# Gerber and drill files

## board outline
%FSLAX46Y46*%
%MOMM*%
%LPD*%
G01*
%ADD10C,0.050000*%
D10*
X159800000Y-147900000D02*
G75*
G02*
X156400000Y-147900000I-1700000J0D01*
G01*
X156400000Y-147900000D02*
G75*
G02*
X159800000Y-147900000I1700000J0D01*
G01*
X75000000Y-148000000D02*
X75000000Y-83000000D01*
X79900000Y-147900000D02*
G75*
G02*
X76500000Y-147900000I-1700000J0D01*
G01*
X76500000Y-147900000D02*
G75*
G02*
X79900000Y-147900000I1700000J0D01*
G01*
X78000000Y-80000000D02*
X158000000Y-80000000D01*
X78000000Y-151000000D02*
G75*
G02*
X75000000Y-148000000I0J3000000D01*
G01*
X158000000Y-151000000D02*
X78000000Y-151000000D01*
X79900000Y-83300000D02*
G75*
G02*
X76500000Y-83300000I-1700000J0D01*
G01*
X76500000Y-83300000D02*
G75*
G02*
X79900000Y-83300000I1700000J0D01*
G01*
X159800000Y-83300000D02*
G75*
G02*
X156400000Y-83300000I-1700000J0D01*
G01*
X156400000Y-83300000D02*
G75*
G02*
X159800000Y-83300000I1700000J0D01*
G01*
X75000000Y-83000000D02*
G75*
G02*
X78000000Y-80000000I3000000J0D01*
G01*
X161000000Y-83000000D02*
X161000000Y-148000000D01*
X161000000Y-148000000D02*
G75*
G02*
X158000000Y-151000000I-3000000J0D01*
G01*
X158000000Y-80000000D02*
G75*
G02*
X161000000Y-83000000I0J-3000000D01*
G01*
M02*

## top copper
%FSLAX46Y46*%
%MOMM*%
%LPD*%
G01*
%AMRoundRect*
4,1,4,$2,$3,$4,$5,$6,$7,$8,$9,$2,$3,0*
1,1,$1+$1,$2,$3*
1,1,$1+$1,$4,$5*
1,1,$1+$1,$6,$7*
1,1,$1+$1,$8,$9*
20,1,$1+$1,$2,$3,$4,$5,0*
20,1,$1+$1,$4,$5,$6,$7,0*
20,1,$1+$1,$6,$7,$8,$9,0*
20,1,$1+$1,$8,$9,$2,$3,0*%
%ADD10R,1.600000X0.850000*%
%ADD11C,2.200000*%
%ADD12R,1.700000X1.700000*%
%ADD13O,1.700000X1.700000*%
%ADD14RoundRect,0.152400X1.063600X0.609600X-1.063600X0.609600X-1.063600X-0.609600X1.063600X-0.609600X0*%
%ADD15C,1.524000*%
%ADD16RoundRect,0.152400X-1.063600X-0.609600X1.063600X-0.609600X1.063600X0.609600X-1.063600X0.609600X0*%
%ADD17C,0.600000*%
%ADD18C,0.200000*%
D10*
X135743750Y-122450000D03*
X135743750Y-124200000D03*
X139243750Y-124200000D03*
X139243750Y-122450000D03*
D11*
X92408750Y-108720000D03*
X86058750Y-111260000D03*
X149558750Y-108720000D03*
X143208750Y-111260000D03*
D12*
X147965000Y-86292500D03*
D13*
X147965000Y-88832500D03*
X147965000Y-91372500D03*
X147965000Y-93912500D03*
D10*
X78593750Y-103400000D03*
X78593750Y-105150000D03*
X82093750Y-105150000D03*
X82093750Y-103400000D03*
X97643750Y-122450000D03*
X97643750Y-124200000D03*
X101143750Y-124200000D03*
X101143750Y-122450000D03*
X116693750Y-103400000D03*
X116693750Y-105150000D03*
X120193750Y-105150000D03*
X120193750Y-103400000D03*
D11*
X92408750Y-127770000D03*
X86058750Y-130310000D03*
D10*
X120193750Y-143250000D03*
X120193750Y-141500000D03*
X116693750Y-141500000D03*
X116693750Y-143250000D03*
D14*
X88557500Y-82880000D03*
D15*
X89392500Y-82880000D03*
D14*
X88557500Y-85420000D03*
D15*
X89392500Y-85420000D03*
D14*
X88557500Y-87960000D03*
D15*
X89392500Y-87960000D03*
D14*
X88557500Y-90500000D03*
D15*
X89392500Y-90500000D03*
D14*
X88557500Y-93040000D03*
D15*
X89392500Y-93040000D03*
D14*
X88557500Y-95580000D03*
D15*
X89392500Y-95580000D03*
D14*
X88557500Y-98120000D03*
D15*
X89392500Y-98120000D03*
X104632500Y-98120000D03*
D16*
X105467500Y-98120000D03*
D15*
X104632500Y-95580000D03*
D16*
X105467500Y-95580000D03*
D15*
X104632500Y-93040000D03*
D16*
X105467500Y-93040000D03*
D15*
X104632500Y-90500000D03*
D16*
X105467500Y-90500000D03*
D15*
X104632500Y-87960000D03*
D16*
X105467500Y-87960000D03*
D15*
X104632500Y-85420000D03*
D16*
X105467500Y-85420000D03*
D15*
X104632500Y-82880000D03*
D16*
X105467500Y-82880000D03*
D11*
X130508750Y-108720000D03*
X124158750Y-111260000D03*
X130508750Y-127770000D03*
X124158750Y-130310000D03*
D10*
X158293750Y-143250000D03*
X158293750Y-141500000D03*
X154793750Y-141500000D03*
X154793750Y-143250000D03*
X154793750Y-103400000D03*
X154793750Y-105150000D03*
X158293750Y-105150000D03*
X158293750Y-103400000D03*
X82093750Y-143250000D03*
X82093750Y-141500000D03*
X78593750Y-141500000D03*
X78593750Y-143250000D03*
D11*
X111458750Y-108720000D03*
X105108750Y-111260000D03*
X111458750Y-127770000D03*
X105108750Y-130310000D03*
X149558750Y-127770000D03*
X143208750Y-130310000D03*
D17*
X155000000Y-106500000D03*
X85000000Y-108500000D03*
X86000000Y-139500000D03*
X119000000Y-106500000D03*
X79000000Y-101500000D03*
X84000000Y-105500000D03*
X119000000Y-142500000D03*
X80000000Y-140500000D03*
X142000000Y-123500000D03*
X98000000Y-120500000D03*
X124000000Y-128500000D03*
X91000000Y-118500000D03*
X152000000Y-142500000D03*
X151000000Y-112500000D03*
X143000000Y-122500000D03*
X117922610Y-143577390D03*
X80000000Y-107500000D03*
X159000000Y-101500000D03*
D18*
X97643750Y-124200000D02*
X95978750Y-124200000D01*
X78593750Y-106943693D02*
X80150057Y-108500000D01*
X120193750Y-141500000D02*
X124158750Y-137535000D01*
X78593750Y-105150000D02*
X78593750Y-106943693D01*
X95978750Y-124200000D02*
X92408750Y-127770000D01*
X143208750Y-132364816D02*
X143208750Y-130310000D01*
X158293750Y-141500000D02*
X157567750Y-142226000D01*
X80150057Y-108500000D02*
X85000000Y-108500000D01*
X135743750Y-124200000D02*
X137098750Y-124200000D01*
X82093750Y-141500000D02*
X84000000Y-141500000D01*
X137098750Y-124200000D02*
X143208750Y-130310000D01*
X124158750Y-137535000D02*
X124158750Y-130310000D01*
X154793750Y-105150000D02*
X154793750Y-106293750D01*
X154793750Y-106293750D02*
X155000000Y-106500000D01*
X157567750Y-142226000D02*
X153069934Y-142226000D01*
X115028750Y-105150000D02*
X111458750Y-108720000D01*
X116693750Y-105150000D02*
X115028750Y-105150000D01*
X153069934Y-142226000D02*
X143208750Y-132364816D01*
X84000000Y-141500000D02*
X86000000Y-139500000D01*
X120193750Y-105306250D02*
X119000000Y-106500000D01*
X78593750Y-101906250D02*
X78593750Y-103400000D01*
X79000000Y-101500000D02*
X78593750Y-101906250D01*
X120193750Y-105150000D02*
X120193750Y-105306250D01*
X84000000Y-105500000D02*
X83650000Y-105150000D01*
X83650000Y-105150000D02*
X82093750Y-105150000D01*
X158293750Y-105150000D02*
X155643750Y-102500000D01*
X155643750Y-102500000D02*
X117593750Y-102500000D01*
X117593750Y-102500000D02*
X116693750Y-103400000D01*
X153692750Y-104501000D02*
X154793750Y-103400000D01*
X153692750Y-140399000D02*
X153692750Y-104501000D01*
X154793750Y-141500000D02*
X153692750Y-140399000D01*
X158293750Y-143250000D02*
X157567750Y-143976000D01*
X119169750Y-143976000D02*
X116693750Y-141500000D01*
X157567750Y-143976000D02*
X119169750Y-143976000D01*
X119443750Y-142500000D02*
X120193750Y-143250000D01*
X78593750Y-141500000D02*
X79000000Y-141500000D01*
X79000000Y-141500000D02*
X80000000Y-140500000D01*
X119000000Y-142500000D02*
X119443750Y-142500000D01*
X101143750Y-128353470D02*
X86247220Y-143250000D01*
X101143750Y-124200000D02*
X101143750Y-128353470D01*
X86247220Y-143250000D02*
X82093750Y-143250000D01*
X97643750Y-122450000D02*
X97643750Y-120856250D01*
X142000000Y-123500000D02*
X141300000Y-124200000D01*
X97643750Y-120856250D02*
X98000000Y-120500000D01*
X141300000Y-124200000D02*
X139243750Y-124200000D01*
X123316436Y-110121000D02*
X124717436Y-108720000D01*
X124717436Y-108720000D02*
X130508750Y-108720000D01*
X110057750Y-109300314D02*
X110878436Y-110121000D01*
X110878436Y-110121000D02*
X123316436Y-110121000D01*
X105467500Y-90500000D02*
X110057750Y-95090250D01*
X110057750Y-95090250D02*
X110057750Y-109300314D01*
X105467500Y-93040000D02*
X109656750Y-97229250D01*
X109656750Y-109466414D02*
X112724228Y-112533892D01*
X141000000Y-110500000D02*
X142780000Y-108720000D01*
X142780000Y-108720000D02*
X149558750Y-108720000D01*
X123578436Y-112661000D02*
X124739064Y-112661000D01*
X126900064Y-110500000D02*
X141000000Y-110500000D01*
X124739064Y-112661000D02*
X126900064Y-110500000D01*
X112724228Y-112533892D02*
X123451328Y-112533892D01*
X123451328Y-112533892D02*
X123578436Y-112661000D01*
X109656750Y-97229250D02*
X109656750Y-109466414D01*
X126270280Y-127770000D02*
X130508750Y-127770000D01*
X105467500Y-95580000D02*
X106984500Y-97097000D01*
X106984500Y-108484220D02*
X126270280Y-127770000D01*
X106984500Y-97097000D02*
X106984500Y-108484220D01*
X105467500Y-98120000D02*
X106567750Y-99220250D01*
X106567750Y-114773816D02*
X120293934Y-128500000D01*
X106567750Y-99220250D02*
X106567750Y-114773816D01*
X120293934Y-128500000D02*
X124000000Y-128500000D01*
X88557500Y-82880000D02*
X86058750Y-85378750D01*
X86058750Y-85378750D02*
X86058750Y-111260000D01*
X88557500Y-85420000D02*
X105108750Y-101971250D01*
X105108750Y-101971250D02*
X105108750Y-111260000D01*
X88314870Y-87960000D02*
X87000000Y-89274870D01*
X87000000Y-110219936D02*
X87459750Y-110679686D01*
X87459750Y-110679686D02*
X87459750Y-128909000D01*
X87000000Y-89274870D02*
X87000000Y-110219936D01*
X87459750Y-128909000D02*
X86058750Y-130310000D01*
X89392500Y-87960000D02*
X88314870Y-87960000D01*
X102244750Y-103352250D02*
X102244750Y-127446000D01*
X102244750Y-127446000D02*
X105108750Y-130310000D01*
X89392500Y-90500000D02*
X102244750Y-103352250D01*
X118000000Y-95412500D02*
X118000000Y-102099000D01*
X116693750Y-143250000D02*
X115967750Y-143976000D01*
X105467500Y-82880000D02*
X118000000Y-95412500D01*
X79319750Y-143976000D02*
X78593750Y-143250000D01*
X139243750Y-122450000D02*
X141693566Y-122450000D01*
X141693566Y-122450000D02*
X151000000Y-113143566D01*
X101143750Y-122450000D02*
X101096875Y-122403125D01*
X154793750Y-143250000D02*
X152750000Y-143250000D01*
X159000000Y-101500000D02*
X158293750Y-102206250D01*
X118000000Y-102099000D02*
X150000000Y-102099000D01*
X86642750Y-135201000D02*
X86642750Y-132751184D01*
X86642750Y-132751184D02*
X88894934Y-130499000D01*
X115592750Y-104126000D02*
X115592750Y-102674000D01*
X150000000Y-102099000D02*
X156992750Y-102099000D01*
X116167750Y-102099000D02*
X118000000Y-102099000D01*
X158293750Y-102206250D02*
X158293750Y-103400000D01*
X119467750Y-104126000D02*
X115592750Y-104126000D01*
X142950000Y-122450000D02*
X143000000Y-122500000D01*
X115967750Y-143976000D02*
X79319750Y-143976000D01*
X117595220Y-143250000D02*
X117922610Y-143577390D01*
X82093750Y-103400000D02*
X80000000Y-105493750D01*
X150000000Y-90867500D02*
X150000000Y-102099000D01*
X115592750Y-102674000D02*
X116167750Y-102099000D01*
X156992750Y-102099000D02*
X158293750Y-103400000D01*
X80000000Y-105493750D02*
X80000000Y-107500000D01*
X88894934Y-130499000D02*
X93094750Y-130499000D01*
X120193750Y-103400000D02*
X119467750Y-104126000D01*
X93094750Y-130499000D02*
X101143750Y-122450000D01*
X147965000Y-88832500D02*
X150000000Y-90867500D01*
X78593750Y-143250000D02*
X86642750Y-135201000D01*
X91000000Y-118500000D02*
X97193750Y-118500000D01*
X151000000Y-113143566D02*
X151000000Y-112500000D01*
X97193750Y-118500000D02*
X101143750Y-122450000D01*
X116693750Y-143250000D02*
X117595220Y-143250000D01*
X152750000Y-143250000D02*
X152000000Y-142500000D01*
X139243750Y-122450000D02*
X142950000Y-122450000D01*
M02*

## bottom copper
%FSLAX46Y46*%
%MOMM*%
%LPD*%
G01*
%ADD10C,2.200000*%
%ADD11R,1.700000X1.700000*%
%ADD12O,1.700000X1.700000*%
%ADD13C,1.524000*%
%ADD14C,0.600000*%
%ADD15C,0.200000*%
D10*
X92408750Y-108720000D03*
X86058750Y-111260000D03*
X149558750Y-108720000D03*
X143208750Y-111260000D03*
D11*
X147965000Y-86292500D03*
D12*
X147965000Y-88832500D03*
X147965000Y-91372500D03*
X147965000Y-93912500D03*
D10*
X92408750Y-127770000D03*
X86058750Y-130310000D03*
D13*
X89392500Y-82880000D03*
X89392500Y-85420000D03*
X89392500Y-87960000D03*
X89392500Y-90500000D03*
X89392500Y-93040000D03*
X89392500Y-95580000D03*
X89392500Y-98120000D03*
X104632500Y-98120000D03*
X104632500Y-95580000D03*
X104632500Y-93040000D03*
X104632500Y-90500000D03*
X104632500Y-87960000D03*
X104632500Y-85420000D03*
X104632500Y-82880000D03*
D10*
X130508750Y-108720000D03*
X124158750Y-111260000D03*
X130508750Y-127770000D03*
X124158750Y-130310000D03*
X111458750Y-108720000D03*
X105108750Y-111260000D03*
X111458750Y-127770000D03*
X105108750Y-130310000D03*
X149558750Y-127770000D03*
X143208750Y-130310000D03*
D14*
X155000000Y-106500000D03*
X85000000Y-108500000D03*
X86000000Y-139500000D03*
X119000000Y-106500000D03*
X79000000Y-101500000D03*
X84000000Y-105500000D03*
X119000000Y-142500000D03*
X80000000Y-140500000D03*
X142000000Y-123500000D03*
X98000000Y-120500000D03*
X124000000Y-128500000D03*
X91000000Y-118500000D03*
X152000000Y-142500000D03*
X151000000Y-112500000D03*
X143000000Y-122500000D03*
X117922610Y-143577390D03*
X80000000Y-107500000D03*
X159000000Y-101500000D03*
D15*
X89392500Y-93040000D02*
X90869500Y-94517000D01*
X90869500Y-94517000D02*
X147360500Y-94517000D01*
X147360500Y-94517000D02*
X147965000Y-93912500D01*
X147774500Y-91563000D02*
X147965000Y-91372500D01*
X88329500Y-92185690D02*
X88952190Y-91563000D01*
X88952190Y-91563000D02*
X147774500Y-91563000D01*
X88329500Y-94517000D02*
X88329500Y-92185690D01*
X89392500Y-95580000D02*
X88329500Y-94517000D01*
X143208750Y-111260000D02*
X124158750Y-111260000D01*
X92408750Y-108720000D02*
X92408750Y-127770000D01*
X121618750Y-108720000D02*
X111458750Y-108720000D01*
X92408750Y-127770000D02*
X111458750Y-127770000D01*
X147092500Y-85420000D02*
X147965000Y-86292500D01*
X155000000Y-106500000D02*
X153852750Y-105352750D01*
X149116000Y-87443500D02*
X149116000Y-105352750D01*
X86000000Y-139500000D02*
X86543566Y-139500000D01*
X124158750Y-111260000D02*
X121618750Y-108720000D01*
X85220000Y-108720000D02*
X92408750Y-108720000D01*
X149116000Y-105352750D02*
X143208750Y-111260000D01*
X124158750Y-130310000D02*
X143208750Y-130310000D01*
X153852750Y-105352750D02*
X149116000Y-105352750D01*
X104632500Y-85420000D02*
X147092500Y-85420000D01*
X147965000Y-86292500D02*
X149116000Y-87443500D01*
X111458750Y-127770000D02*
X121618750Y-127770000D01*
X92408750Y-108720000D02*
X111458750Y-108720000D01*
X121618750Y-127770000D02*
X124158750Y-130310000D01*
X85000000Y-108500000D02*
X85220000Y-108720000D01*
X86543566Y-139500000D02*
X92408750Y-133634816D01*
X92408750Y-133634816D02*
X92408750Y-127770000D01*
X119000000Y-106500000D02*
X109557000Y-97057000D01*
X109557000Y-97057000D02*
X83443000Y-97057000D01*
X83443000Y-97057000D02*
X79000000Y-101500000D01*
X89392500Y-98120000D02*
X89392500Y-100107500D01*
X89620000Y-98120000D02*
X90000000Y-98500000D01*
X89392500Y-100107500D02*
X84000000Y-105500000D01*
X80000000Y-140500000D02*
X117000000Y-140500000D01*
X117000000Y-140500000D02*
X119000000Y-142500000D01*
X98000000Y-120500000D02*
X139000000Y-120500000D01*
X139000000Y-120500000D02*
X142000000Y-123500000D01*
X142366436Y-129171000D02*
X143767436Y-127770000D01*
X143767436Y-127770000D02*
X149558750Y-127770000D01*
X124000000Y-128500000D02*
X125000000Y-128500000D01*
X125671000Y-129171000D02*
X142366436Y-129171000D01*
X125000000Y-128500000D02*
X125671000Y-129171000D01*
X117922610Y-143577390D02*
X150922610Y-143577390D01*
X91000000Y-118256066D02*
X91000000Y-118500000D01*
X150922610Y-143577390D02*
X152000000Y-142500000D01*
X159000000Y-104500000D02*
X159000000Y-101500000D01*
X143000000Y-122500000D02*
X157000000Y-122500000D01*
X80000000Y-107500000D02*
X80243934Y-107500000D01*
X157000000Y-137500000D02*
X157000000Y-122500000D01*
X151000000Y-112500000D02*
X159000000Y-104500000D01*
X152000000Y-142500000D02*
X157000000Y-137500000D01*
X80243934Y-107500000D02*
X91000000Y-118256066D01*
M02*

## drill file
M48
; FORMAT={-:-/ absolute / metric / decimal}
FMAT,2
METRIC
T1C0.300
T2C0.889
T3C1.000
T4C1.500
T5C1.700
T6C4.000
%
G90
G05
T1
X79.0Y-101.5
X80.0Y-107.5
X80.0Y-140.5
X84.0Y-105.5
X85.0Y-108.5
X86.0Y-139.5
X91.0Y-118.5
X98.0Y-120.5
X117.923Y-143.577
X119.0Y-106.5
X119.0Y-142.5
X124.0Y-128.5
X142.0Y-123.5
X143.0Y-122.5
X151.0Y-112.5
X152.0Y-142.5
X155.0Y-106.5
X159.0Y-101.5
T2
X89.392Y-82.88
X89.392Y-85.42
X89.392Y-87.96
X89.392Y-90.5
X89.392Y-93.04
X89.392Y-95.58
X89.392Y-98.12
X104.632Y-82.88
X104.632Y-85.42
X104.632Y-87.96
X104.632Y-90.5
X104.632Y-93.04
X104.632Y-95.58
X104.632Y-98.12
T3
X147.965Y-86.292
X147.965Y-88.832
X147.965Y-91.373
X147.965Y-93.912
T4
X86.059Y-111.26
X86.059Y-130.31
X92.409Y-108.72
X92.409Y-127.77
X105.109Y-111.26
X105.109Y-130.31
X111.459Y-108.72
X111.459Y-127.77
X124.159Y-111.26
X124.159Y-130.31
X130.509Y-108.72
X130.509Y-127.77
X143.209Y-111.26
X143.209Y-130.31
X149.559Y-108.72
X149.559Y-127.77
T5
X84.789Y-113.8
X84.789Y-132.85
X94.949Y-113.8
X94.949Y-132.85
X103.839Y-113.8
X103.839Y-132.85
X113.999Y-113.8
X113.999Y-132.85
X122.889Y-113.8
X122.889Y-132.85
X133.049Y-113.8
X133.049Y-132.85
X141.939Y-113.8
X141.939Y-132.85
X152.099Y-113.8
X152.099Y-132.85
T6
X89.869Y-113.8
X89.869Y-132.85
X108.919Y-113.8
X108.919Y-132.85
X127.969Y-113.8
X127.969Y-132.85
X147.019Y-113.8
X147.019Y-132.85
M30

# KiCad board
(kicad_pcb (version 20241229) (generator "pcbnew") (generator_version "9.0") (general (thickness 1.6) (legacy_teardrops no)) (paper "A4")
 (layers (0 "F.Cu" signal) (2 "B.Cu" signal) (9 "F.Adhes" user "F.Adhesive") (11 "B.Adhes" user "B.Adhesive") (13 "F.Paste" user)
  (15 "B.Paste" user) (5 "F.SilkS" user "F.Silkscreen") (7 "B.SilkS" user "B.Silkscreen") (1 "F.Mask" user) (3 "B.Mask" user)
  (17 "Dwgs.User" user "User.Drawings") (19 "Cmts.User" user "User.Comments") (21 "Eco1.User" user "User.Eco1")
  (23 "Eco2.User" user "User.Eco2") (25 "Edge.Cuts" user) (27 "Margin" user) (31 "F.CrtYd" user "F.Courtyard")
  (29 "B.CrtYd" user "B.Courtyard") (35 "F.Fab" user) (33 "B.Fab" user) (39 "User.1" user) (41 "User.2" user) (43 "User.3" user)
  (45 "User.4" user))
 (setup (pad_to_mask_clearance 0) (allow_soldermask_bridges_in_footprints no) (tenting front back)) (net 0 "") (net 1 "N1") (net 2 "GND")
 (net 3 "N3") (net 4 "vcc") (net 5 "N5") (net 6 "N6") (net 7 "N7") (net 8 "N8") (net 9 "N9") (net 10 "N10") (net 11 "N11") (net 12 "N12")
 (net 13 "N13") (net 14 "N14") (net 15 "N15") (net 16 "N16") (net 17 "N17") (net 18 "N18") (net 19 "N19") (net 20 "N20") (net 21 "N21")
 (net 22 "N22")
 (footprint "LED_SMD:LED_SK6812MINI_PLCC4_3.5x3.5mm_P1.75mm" (layer "F.Cu") (at 137.49375 123.325)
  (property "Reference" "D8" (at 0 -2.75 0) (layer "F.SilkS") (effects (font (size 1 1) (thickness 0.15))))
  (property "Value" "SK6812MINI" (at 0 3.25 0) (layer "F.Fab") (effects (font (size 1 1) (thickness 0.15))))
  (pad "1" smd rect (at -1.75 -0.875) (size 1.6 0.85) (layers "F.Cu" "F.Mask" "F.Paste") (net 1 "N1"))
  (pad "2" smd rect (at -1.75 0.875) (size 1.6 0.85) (layers "F.Cu" "F.Mask" "F.Paste") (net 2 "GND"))
  (pad "3" smd rect (at 1.75 0.875) (size 1.6 0.85) (layers "F.Cu" "F.Mask" "F.Paste") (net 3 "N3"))
  (pad "4" smd rect (at 1.75 -0.875) (size 1.6 0.85) (layers "F.Cu" "F.Mask" "F.Paste") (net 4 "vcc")))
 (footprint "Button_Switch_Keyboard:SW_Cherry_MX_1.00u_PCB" (layer "F.Cu") (at 92.40875 108.72)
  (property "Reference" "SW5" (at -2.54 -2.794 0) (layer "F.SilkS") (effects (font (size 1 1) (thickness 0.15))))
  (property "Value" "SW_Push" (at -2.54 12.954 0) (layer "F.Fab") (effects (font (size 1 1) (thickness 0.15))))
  (pad "" np_thru_hole circle (at -7.62 5.08) (size 1.7 1.7) (drill 1.7) (layers "*.Cu" "*.Mask"))
  (pad "" np_thru_hole circle (at -2.54 5.08) (size 4 4) (drill 4) (layers "*.Cu" "*.Mask"))
  (pad "" np_thru_hole circle (at 2.54 5.08) (size 1.7 1.7) (drill 1.7) (layers "*.Cu" "*.Mask"))
  (pad "1" thru_hole circle (at 0 0) (size 2.2 2.2) (drill 1.5) (layers "*.Cu" "*.Mask") (remove_unused_layers no) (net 2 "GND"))
  (pad "2" thru_hole circle (at -6.35 2.54) (size 2.2 2.2) (drill 1.5) (layers "*.Cu" "*.Mask") (remove_unused_layers no) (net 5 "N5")))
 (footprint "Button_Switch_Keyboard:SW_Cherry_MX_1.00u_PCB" (layer "F.Cu") (at 149.55875 108.72)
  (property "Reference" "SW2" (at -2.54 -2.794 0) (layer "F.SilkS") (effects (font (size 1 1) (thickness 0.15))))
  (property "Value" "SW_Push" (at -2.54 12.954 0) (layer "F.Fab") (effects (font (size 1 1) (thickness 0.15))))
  (pad "" np_thru_hole circle (at -7.62 5.08) (size 1.7 1.7) (drill 1.7) (layers "*.Cu" "*.Mask"))
  (pad "" np_thru_hole circle (at -2.54 5.08) (size 4 4) (drill 4) (layers "*.Cu" "*.Mask"))
  (pad "" np_thru_hole circle (at 2.54 5.08) (size 1.7 1.7) (drill 1.7) (layers "*.Cu" "*.Mask"))
  (pad "1" thru_hole circle (at 0 0) (size 2.2 2.2) (drill 1.5) (layers "*.Cu" "*.Mask") (remove_unused_layers no) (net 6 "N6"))
  (pad "2" thru_hole circle (at -6.35 2.54) (size 2.2 2.2) (drill 1.5) (layers "*.Cu" "*.Mask") (remove_unused_layers no) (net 2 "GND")))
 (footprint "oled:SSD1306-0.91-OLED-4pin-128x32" (layer "F.Cu") (at 111.465 84.1025)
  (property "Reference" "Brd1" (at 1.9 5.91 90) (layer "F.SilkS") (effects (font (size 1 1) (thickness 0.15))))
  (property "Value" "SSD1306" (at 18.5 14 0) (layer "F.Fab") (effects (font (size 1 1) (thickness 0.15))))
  (pad "1" thru_hole rect (at 36.5 2.19) (size 1.7 1.7) (drill 1) (layers "*.Cu" "*.Mask") (remove_unused_layers no) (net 2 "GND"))
  (pad "2" thru_hole oval (at 36.5 4.73) (size 1.7 1.7) (drill 1) (layers "*.Cu" "*.Mask") (remove_unused_layers no) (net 4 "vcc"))
  (pad "3" thru_hole oval (at 36.5 7.27) (size 1.7 1.7) (drill 1) (layers "*.Cu" "*.Mask") (remove_unused_layers no) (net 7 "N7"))
  (pad "4" thru_hole oval (at 36.5 9.81) (size 1.7 1.7) (drill 1) (layers "*.Cu" "*.Mask") (remove_unused_layers no) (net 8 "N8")))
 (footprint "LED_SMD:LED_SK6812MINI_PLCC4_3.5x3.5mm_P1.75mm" (layer "F.Cu") (at 80.34375 104.275)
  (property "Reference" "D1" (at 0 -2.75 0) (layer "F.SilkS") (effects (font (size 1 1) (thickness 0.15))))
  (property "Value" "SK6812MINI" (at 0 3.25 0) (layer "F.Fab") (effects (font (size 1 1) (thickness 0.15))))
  (pad "1" smd rect (at -1.75 -0.875) (size 1.6 0.85) (layers "F.Cu" "F.Mask" "F.Paste") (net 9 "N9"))
  (pad "2" smd rect (at -1.75 0.875) (size 1.6 0.85) (layers "F.Cu" "F.Mask" "F.Paste") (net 2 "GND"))
  (pad "3" smd rect (at 1.75 0.875) (size 1.6 0.85) (layers "F.Cu" "F.Mask" "F.Paste") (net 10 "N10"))
  (pad "4" smd rect (at 1.75 -0.875) (size 1.6 0.85) (layers "F.Cu" "F.Mask" "F.Paste") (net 4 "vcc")))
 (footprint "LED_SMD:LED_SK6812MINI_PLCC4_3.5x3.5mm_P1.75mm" (layer "F.Cu") (at 99.39375 123.325)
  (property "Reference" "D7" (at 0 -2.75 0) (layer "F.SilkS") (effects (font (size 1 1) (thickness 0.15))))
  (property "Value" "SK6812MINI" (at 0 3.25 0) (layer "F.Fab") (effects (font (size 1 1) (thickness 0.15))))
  (pad "1" smd rect (at -1.75 -0.875) (size 1.6 0.85) (layers "F.Cu" "F.Mask" "F.Paste") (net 3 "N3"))
  (pad "2" smd rect (at -1.75 0.875) (size 1.6 0.85) (layers "F.Cu" "F.Mask" "F.Paste") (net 2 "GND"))
  (pad "3" smd rect (at 1.75 0.875) (size 1.6 0.85) (layers "F.Cu" "F.Mask" "F.Paste") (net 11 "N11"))
  (pad "4" smd rect (at 1.75 -0.875) (size 1.6 0.85) (layers "F.Cu" "F.Mask" "F.Paste") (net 4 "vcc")))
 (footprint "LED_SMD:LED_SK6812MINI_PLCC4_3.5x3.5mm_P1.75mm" (layer "F.Cu") (at 118.44375 104.275)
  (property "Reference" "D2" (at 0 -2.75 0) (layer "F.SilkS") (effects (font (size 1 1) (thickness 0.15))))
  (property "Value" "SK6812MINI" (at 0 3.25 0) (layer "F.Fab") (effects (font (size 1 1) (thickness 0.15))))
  (pad "1" smd rect (at -1.75 -0.875) (size 1.6 0.85) (layers "F.Cu" "F.Mask" "F.Paste") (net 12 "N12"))
  (pad "2" smd rect (at -1.75 0.875) (size 1.6 0.85) (layers "F.Cu" "F.Mask" "F.Paste") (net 2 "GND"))
  (pad "3" smd rect (at 1.75 0.875) (size 1.6 0.85) (layers "F.Cu" "F.Mask" "F.Paste") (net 9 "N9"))
  (pad "4" smd rect (at 1.75 -0.875) (size 1.6 0.85) (layers "F.Cu" "F.Mask" "F.Paste") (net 4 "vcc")))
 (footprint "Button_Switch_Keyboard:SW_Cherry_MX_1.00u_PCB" (layer "F.Cu") (at 92.40875 127.77)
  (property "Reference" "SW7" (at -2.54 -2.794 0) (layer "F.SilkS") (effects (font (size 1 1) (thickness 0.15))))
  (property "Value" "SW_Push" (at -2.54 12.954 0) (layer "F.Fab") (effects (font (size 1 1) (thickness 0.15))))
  (pad "" np_thru_hole circle (at -7.62 5.08) (size 1.7 1.7) (drill 1.7) (layers "*.Cu" "*.Mask"))
  (pad "" np_thru_hole circle (at -2.54 5.08) (size 4 4) (drill 4) (layers "*.Cu" "*.Mask"))
  (pad "" np_thru_hole circle (at 2.54 5.08) (size 1.7 1.7) (drill 1.7) (layers "*.Cu" "*.Mask"))
  (pad "1" thru_hole circle (at 0 0) (size 2.2 2.2) (drill 1.5) (layers "*.Cu" "*.Mask") (remove_unused_layers no) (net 2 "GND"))
  (pad "2" thru_hole circle (at -6.35 2.54) (size 2.2 2.2) (drill 1.5) (layers "*.Cu" "*.Mask") (remove_unused_layers no) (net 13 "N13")))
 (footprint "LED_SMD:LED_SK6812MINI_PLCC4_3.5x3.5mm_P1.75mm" (layer "F.Cu") (at 118.44375 142.375 180)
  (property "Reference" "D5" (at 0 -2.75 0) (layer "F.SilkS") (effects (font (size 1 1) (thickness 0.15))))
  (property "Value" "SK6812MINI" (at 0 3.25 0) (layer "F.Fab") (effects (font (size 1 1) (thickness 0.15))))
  (pad "1" smd rect (at -1.75 -0.875 180) (size 1.6 0.85) (layers "F.Cu" "F.Mask" "F.Paste") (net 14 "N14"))
  (pad "2" smd rect (at -1.75 0.875 180) (size 1.6 0.85) (layers "F.Cu" "F.Mask" "F.Paste") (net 2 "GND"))
  (pad "3" smd rect (at 1.75 0.875 180) (size 1.6 0.85) (layers "F.Cu" "F.Mask" "F.Paste") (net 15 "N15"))
  (pad "4" smd rect (at 1.75 -0.875 180) (size 1.6 0.85) (layers "F.Cu" "F.Mask" "F.Paste") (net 4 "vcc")))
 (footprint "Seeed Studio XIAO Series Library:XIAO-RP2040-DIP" (layer "F.Cu") (at 97.0125 90.5)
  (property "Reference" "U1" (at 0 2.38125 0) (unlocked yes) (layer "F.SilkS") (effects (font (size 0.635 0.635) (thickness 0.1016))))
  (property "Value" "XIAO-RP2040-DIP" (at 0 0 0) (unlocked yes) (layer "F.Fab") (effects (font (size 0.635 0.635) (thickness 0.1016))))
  (pad "1" smd roundrect (at -8.455 -7.62 180) (size 2.432 1.524) (layers "F.Cu" "F.Mask") (roundrect_rratio 0.1) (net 5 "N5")
   (thermal_bridge_angle 45))
  (pad "1" thru_hole circle (at -7.62 -7.62 180) (size 1.524 1.524) (drill 0.889) (layers "*.Cu" "*.Mask") (remove_unused_layers no)
   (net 5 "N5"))
  (pad "2" smd roundrect (at -8.455 -5.08 180) (size 2.432 1.524) (layers "F.Cu" "F.Mask") (roundrect_rratio 0.1) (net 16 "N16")
   (thermal_bridge_angle 45))
  (pad "2" thru_hole circle (at -7.62 -5.08 180) (size 1.524 1.524) (drill 0.889) (layers "*.Cu" "*.Mask") (remove_unused_layers no)
   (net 16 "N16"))
  (pad "3" smd roundrect (at -8.455 -2.54 180) (size 2.432 1.524) (layers "F.Cu" "F.Mask") (roundrect_rratio 0.1) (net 13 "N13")
   (thermal_bridge_angle 45))
  (pad "3" thru_hole circle (at -7.62 -2.54 180) (size 1.524 1.524) (drill 0.889) (layers "*.Cu" "*.Mask") (remove_unused_layers no)
   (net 13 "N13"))
  (pad "4" smd roundrect (at -8.455 0 180) (size 2.432 1.524) (layers "F.Cu" "F.Mask") (roundrect_rratio 0.1) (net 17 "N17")
   (thermal_bridge_angle 45))
  (pad "4" thru_hole circle (at -7.62 0 180) (size 1.524 1.524) (drill 0.889) (layers "*.Cu" "*.Mask") (remove_unused_layers no)
   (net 17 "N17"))
  (pad "5" smd roundrect (at -8.455 2.54 180) (size 2.432 1.524) (layers "F.Cu" "F.Mask") (roundrect_rratio 0.1) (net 8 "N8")
   (thermal_bridge_angle 45))
  (pad "5" thru_hole circle (at -7.62 2.54 180) (size 1.524 1.524) (drill 0.889) (layers "*.Cu" "*.Mask") (remove_unused_layers no)
   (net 8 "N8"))
  (pad "6" smd roundrect (at -8.455 5.08 180) (size 2.432 1.524) (layers "F.Cu" "F.Mask") (roundrect_rratio 0.1) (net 7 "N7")
   (thermal_bridge_angle 45))
  (pad "6" thru_hole circle (at -7.62 5.08 180) (size 1.524 1.524) (drill 0.889) (layers "*.Cu" "*.Mask") (remove_unused_layers no)
   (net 7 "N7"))
  (pad "7" smd roundrect (at -8.455 7.62 180) (size 2.432 1.524) (layers "F.Cu" "F.Mask") (roundrect_rratio 0.1) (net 10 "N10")
   (thermal_bridge_angle 45))
  (pad "7" thru_hole circle (at -7.62 7.62 180) (size 1.524 1.524) (drill 0.889) (layers "*.Cu" "*.Mask") (remove_unused_layers no)
   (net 10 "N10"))
  (pad "8" thru_hole circle (at 7.62 7.62) (size 1.524 1.524) (drill 0.889) (layers "*.Cu" "*.Mask") (remove_unused_layers no)
   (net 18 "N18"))
  (pad "8" smd roundrect (at 8.455 7.62) (size 2.432 1.524) (layers "F.Cu" "F.Mask") (roundrect_rratio 0.1) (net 18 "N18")
   (thermal_bridge_angle 45))
  (pad "9" thru_hole circle (at 7.62 5.08) (size 1.524 1.524) (drill 0.889) (layers "*.Cu" "*.Mask") (remove_unused_layers no)
   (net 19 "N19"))
  (pad "9" smd roundrect (at 8.455 5.08) (size 2.432 1.524) (layers "F.Cu" "F.Mask") (roundrect_rratio 0.1) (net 19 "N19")
   (thermal_bridge_angle 45))
  (pad "10" thru_hole circle (at 7.62 2.54) (size 1.524 1.524) (drill 0.889) (layers "*.Cu" "*.Mask") (remove_unused_layers no) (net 6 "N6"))
  (pad "10" smd roundrect (at 8.455 2.54) (size 2.432 1.524) (layers "F.Cu" "F.Mask") (roundrect_rratio 0.1) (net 6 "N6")
   (thermal_bridge_angle 45))
  (pad "11" thru_hole circle (at 7.62 0) (size 1.524 1.524) (drill 0.889) (layers "*.Cu" "*.Mask") (remove_unused_layers no) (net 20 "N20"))
  (pad "11" smd roundrect (at 8.455 0) (size 2.432 1.524) (layers "F.Cu" "F.Mask") (roundrect_rratio 0.1) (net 20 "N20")
   (thermal_bridge_angle 45))
  (pad "12" thru_hole circle (at 7.62 -2.54) (size 1.524 1.524) (drill 0.889) (layers "*.Cu" "*.Mask") (remove_unused_layers no)
   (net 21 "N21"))
  (pad "12" smd roundrect (at 8.455 -2.54) (size 2.432 1.524) (layers "F.Cu" "F.Mask") (roundrect_rratio 0.1) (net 21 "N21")
   (thermal_bridge_angle 45))
  (pad "13" thru_hole circle (at 7.62 -5.08) (size 1.524 1.524) (drill 0.889) (layers "*.Cu" "*.Mask") (remove_unused_layers no)
   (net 2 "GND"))
  (pad "13" smd roundrect (at 8.455 -5.08) (size 2.432 1.524) (layers "F.Cu" "F.Mask") (roundrect_rratio 0.1) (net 2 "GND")
   (thermal_bridge_angle 45))
  (pad "14" thru_hole circle (at 7.62 -7.62) (size 1.524 1.524) (drill 0.889) (layers "*.Cu" "*.Mask") (remove_unused_layers no)
   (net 4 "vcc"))
  (pad "14" smd roundrect (at 8.455 -7.62) (size 2.432 1.524) (layers "F.Cu" "F.Mask") (roundrect_rratio 0.1) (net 4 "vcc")
   (thermal_bridge_angle 45)))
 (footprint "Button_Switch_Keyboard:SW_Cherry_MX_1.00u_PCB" (layer "F.Cu") (at 130.50875 108.72)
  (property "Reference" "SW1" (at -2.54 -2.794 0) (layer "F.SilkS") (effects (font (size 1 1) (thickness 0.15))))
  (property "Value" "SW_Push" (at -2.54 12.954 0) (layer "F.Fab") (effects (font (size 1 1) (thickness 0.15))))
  (pad "" np_thru_hole circle (at -7.62 5.08) (size 1.7 1.7) (drill 1.7) (layers "*.Cu" "*.Mask"))
  (pad "" np_thru_hole circle (at -2.54 5.08) (size 4 4) (drill 4) (layers "*.Cu" "*.Mask"))
  (pad "" np_thru_hole circle (at 2.54 5.08) (size 1.7 1.7) (drill 1.7) (layers "*.Cu" "*.Mask"))
  (pad "1" thru_hole circle (at 0 0) (size 2.2 2.2) (drill 1.5) (layers "*.Cu" "*.Mask") (remove_unused_layers no) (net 20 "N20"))
  (pad "2" thru_hole circle (at -6.35 2.54) (size 2.2 2.2) (drill 1.5) (layers "*.Cu" "*.Mask") (remove_unused_layers no) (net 2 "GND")))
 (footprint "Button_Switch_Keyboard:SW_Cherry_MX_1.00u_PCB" (layer "F.Cu") (at 130.50875 127.77)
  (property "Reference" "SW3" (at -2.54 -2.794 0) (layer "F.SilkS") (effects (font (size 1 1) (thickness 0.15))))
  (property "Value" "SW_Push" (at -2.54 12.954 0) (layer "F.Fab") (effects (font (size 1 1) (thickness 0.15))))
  (pad "" np_thru_hole circle (at -7.62 5.08) (size 1.7 1.7) (drill 1.7) (layers "*.Cu" "*.Mask"))
  (pad "" np_thru_hole circle (at -2.54 5.08) (size 4 4) (drill 4) (layers "*.Cu" "*.Mask"))
  (pad "" np_thru_hole circle (at 2.54 5.08) (size 1.7 1.7) (drill 1.7) (layers "*.Cu" "*.Mask"))
  (pad "1" thru_hole circle (at 0 0) (size 2.2 2.2) (drill 1.5) (layers "*.Cu" "*.Mask") (remove_unused_layers no) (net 19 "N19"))
  (pad "2" thru_hole circle (at -6.35 2.54) (size 2.2 2.2) (drill 1.5) (layers "*.Cu" "*.Mask") (remove_unused_layers no) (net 2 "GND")))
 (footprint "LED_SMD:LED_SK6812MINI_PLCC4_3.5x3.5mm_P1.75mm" (layer "F.Cu") (at 156.54375 142.375 180)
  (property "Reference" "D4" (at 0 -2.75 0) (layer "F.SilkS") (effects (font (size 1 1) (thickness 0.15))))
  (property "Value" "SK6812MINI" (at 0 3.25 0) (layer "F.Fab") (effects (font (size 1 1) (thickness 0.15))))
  (pad "1" smd rect (at -1.75 -0.875 180) (size 1.6 0.85) (layers "F.Cu" "F.Mask" "F.Paste") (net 15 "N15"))
  (pad "2" smd rect (at -1.75 0.875 180) (size 1.6 0.85) (layers "F.Cu" "F.Mask" "F.Paste") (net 2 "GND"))
  (pad "3" smd rect (at 1.75 0.875 180) (size 1.6 0.85) (layers "F.Cu" "F.Mask" "F.Paste") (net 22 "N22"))
  (pad "4" smd rect (at 1.75 -0.875 180) (size 1.6 0.85) (layers "F.Cu" "F.Mask" "F.Paste") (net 4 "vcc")))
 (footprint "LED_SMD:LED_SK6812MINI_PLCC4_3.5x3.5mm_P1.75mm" (layer "F.Cu") (at 156.54375 104.275)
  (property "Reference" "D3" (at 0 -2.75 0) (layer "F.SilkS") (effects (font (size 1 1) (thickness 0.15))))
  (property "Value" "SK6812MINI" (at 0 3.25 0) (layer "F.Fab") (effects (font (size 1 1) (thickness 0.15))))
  (pad "1" smd rect (at -1.75 -0.875) (size 1.6 0.85) (layers "F.Cu" "F.Mask" "F.Paste") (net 22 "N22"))
  (pad "2" smd rect (at -1.75 0.875) (size 1.6 0.85) (layers "F.Cu" "F.Mask" "F.Paste") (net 2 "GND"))
  (pad "3" smd rect (at 1.75 0.875) (size 1.6 0.85) (layers "F.Cu" "F.Mask" "F.Paste") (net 12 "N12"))
  (pad "4" smd rect (at 1.75 -0.875) (size 1.6 0.85) (layers "F.Cu" "F.Mask" "F.Paste") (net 4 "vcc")))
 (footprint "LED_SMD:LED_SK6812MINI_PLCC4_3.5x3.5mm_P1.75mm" (layer "F.Cu") (at 80.34375 142.375 180)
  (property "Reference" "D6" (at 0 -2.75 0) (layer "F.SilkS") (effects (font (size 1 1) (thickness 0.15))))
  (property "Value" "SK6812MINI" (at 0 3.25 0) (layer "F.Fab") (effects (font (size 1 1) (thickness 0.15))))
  (pad "1" smd rect (at -1.75 -0.875 180) (size 1.6 0.85) (layers "F.Cu" "F.Mask" "F.Paste") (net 11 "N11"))
  (pad "2" smd rect (at -1.75 0.875 180) (size 1.6 0.85) (layers "F.Cu" "F.Mask" "F.Paste") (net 2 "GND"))
  (pad "3" smd rect (at 1.75 0.875 180) (size 1.6 0.85) (layers "F.Cu" "F.Mask" "F.Paste") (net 14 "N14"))
  (pad "4" smd rect (at 1.75 -0.875 180) (size 1.6 0.85) (layers "F.Cu" "F.Mask" "F.Paste") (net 4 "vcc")))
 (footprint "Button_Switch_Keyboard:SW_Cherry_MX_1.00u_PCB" (layer "F.Cu") (at 111.45875 108.72)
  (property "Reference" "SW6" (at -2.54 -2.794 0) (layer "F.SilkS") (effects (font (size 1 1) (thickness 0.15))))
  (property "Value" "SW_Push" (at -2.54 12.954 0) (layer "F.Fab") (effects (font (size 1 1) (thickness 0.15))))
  (pad "" np_thru_hole circle (at -7.62 5.08) (size 1.7 1.7) (drill 1.7) (layers "*.Cu" "*.Mask"))
  (pad "" np_thru_hole circle (at -2.54 5.08) (size 4 4) (drill 4) (layers "*.Cu" "*.Mask"))
  (pad "" np_thru_hole circle (at 2.54 5.08) (size 1.7 1.7) (drill 1.7) (layers "*.Cu" "*.Mask"))
  (pad "1" thru_hole circle (at 0 0) (size 2.2 2.2) (drill 1.5) (layers "*.Cu" "*.Mask") (remove_unused_layers no) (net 2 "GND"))
  (pad "2" thru_hole circle (at -6.35 2.54) (size 2.2 2.2) (drill 1.5) (layers "*.Cu" "*.Mask") (remove_unused_layers no) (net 16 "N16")))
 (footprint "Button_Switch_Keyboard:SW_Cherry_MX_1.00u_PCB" (layer "F.Cu") (at 111.45875 127.77)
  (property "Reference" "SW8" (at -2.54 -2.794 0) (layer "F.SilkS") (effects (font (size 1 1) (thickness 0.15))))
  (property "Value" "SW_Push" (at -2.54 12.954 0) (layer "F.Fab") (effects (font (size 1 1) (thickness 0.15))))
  (pad "" np_thru_hole circle (at -7.62 5.08) (size 1.7 1.7) (drill 1.7) (layers "*.Cu" "*.Mask"))
  (pad "" np_thru_hole circle (at -2.54 5.08) (size 4 4) (drill 4) (layers "*.Cu" "*.Mask"))
  (pad "" np_thru_hole circle (at 2.54 5.08) (size 1.7 1.7) (drill 1.7) (layers "*.Cu" "*.Mask"))
  (pad "1" thru_hole circle (at 0 0) (size 2.2 2.2) (drill 1.5) (layers "*.Cu" "*.Mask") (remove_unused_layers no) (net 2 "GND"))
  (pad "2" thru_hole circle (at -6.35 2.54) (size 2.2 2.2) (drill 1.5) (layers "*.Cu" "*.Mask") (remove_unused_layers no) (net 17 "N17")))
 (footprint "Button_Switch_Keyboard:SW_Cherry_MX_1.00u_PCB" (layer "F.Cu") (at 149.55875 127.77)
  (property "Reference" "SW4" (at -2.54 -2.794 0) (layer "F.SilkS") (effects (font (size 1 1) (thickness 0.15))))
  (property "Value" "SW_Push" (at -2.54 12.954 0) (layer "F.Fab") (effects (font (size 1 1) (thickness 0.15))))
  (pad "" np_thru_hole circle (at -7.62 5.08) (size 1.7 1.7) (drill 1.7) (layers "*.Cu" "*.Mask"))
  (pad "" np_thru_hole circle (at -2.54 5.08) (size 4 4) (drill 4) (layers "*.Cu" "*.Mask"))
  (pad "" np_thru_hole circle (at 2.54 5.08) (size 1.7 1.7) (drill 1.7) (layers "*.Cu" "*.Mask"))
  (pad "1" thru_hole circle (at 0 0) (size 2.2 2.2) (drill 1.5) (layers "*.Cu" "*.Mask") (remove_unused_layers no) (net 18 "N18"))
  (pad "2" thru_hole circle (at -6.35 2.54) (size 2.2 2.2) (drill 1.5) (layers "*.Cu" "*.Mask") (remove_unused_layers no) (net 2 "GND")))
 (gr_circle (center 158.1 147.9) (end 159.8 147.9) (stroke (width 0.05) (type default)) (fill no) (layer "Edge.Cuts"))
 (gr_line (start 75 148) (end 75 83) (stroke (width 0.05) (type default)) (layer "Edge.Cuts"))
 (gr_circle (center 78.2 147.9) (end 79.9 147.9) (stroke (width 0.05) (type default)) (fill no) (layer "Edge.Cuts"))
 (gr_line (start 78 80) (end 158 80) (stroke (width 0.05) (type default)) (layer "Edge.Cuts"))
 (gr_arc (start 78 151) (mid 75.87868 150.12132) (end 75 148) (stroke (width 0.05) (type default)) (layer "Edge.Cuts"))
 (gr_line (start 158 151) (end 78 151) (stroke (width 0.05) (type default)) (layer "Edge.Cuts"))
 (gr_circle (center 78.2 83.3) (end 79.9 83.3) (stroke (width 0.05) (type default)) (fill no) (layer "Edge.Cuts"))
 (gr_circle (center 158.1 83.3) (end 158.1 81.6) (stroke (width 0.05) (type default)) (fill no) (layer "Edge.Cuts"))
 (gr_arc (start 75 83) (mid 75.87868 80.87868) (end 78 80) (stroke (width 0.05) (type default)) (layer "Edge.Cuts"))
 (gr_line (start 161 83) (end 161 148) (stroke (width 0.05) (type default)) (layer "Edge.Cuts"))
 (gr_arc (start 161 148) (mid 160.12132 150.12132) (end 158 151) (stroke (width 0.05) (type default)) (layer "Edge.Cuts"))
 (gr_arc (start 158 80) (mid 160.12132 80.87868) (end 161 83) (stroke (width 0.05) (type default)) (layer "Edge.Cuts"))
 (segment (start 89.3925 93.04) (end 90.8695 94.517) (width 0.2) (layer "B.Cu") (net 8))
 (segment (start 90.8695 94.517) (end 147.3605 94.517) (width 0.2) (layer "B.Cu") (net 8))
 (segment (start 147.3605 94.517) (end 147.965 93.9125) (width 0.2) (layer "B.Cu") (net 8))
 (segment (start 147.7745 91.563) (end 147.965 91.3725) (width 0.2) (layer "B.Cu") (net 7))
 (segment (start 88.3295 92.18569) (end 88.95219 91.563) (width 0.2) (layer "B.Cu") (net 7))
 (segment (start 88.95219 91.563) (end 147.7745 91.563) (width 0.2) (layer "B.Cu") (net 7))
 (segment (start 88.3295 94.517) (end 88.3295 92.18569) (width 0.2) (layer "B.Cu") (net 7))
 (segment (start 89.3925 95.58) (end 88.3295 94.517) (width 0.2) (layer "B.Cu") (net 7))
 (segment (start 97.64375 124.2) (end 95.97875 124.2) (width 0.2) (layer "F.Cu") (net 2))
 (segment (start 78.59375 106.943693) (end 80.150057 108.5) (width 0.2) (layer "F.Cu") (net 2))
 (segment (start 120.19375 141.5) (end 124.15875 137.535) (width 0.2) (layer "F.Cu") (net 2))
 (segment (start 78.59375 105.15) (end 78.59375 106.943693) (width 0.2) (layer "F.Cu") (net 2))
 (segment (start 95.97875 124.2) (end 92.40875 127.77) (width 0.2) (layer "F.Cu") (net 2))
 (segment (start 143.20875 132.364816) (end 143.20875 130.31) (width 0.2) (layer "F.Cu") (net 2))
 (segment (start 158.29375 141.5) (end 157.56775 142.226) (width 0.2) (layer "F.Cu") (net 2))
 (segment (start 80.150057 108.5) (end 85 108.5) (width 0.2) (layer "F.Cu") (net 2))
 (segment (start 135.74375 124.2) (end 137.09875 124.2) (width 0.2) (layer "F.Cu") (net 2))
 (segment (start 82.09375 141.5) (end 84 141.5) (width 0.2) (layer "F.Cu") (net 2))
 (segment (start 137.09875 124.2) (end 143.20875 130.31) (width 0.2) (layer "F.Cu") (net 2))
 (segment (start 124.15875 137.535) (end 124.15875 130.31) (width 0.2) (layer "F.Cu") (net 2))
 (segment (start 154.79375 105.15) (end 154.79375 106.29375) (width 0.2) (layer "F.Cu") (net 2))
 (segment (start 154.79375 106.29375) (end 155 106.5) (width 0.2) (layer "F.Cu") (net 2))
 (segment (start 157.56775 142.226) (end 153.069934 142.226) (width 0.2) (layer "F.Cu") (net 2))
 (segment (start 115.02875 105.15) (end 111.45875 108.72) (width 0.2) (layer "F.Cu") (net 2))
 (segment (start 116.69375 105.15) (end 115.02875 105.15) (width 0.2) (layer "F.Cu") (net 2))
 (segment (start 153.069934 142.226) (end 143.20875 132.364816) (width 0.2) (layer "F.Cu") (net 2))
 (segment (start 84 141.5) (end 86 139.5) (width 0.2) (layer "F.Cu") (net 2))
 (via (at 155 106.5) (size 0.6) (drill 0.3) (layers "F.Cu" "B.Cu") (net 2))
 (via (at 85 108.5) (size 0.6) (drill 0.3) (layers "F.Cu" "B.Cu") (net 2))
 (via (at 86 139.5) (size 0.6) (drill 0.3) (layers "F.Cu" "B.Cu") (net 2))
 (segment (start 143.20875 111.26) (end 124.15875 111.26) (width 0.2) (layer "B.Cu") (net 2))
 (segment (start 92.40875 108.72) (end 92.40875 127.77) (width 0.2) (layer "B.Cu") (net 2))
 (segment (start 121.61875 108.72) (end 111.45875 108.72) (width 0.2) (layer "B.Cu") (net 2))
 (segment (start 92.40875 127.77) (end 111.45875 127.77) (width 0.2) (layer "B.Cu") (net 2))
 (segment (start 147.0925 85.42) (end 147.965 86.2925) (width 0.2) (layer "B.Cu") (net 2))
 (segment (start 155 106.5) (end 153.85275 105.35275) (width 0.2) (layer "B.Cu") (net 2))
 (segment (start 149.116 87.4435) (end 149.116 105.35275) (width 0.2) (layer "B.Cu") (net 2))
 (segment (start 86 139.5) (end 86.543566 139.5) (width 0.2) (layer "B.Cu") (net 2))
 (segment (start 124.15875 111.26) (end 121.61875 108.72) (width 0.2) (layer "B.Cu") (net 2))
 (segment (start 85.22 108.72) (end 92.40875 108.72) (width 0.2) (layer "B.Cu") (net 2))
 (segment (start 149.116 105.35275) (end 143.20875 111.26) (width 0.2) (layer "B.Cu") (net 2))
 (segment (start 124.15875 130.31) (end 143.20875 130.31) (width 0.2) (layer "B.Cu") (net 2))
 (segment (start 153.85275 105.35275) (end 149.116 105.35275) (width 0.2) (layer "B.Cu") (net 2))
 (segment (start 104.6325 85.42) (end 147.0925 85.42) (width 0.2) (layer "B.Cu") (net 2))
 (segment (start 147.965 86.2925) (end 149.116 87.4435) (width 0.2) (layer "B.Cu") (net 2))
 (segment (start 111.45875 127.77) (end 121.61875 127.77) (width 0.2) (layer "B.Cu") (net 2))
 (segment (start 92.40875 108.72) (end 111.45875 108.72) (width 0.2) (layer "B.Cu") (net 2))
 (segment (start 121.61875 127.77) (end 124.15875 130.31) (width 0.2) (layer "B.Cu") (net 2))
 (segment (start 85 108.5) (end 85.22 108.72) (width 0.2) (layer "B.Cu") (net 2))
 (segment (start 86.543566 139.5) (end 92.40875 133.634816) (width 0.2) (layer "B.Cu") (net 2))
 (segment (start 92.40875 133.634816) (end 92.40875 127.77) (width 0.2) (layer "B.Cu") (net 2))
 (segment (start 120.19375 105.30625) (end 119 106.5) (width 0.2) (layer "F.Cu") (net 9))
 (segment (start 78.59375 101.90625) (end 78.59375 103.4) (width 0.2) (layer "F.Cu") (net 9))
 (segment (start 79 101.5) (end 78.59375 101.90625) (width 0.2) (layer "F.Cu") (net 9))
 (segment (start 120.19375 105.15) (end 120.19375 105.30625) (width 0.2) (layer "F.Cu") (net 9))
 (via (at 119 106.5) (size 0.6) (drill 0.3) (layers "F.Cu" "B.Cu") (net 9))
 (via (at 79 101.5) (size 0.6) (drill 0.3) (layers "F.Cu" "B.Cu") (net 9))
 (segment (start 119 106.5) (end 109.557 97.057) (width 0.2) (layer "B.Cu") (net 9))
 (segment (start 109.557 97.057) (end 83.443 97.057) (width 0.2) (layer "B.Cu") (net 9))
 (segment (start 83.443 97.057) (end 79 101.5) (width 0.2) (layer "B.Cu") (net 9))
 (segment (start 84 105.5) (end 83.65 105.15) (width 0.2) (layer "F.Cu") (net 10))
 (segment (start 83.65 105.15) (end 82.09375 105.15) (width 0.2) (layer "F.Cu") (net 10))
 (via (at 84 105.5) (size 0.6) (drill 0.3) (layers "F.Cu" "B.Cu") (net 10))
 (segment (start 89.3925 98.12) (end 89.3925 100.1075) (width 0.2) (layer "B.Cu") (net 10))
 (segment (start 89.62 98.12) (end 90 98.5) (width 0.2) (layer "B.Cu") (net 10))
 (segment (start 89.3925 100.1075) (end 84 105.5) (width 0.2) (layer "B.Cu") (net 10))
 (segment (start 158.29375 105.15) (end 155.64375 102.5) (width 0.2) (layer "F.Cu") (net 12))
 (segment (start 155.64375 102.5) (end 117.59375 102.5) (width 0.2) (layer "F.Cu") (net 12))
 (segment (start 117.59375 102.5) (end 116.69375 103.4) (width 0.2) (layer "F.Cu") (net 12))
 (segment (start 153.69275 104.501) (end 154.79375 103.4) (width 0.2) (layer "F.Cu") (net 22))
 (segment (start 153.69275 140.399) (end 153.69275 104.501) (width 0.2) (layer "F.Cu") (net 22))
 (segment (start 154.79375 141.5) (end 153.69275 140.399) (width 0.2) (layer "F.Cu") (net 22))
 (segment (start 158.29375 143.25) (end 157.56775 143.976) (width 0.2) (layer "F.Cu") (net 15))
 (segment (start 119.16975 143.976) (end 116.69375 141.5) (width 0.2) (layer "F.Cu") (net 15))
 (segment (start 157.56775 143.976) (end 119.16975 143.976) (width 0.2) (layer "F.Cu") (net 15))
 (segment (start 119.44375 142.5) (end 120.19375 143.25) (width 0.2) (layer "F.Cu") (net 14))
 (segment (start 78.59375 141.5) (end 79 141.5) (width 0.2) (layer "F.Cu") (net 14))
 (segment (start 79 141.5) (end 80 140.5) (width 0.2) (layer "F.Cu") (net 14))
 (segment (start 119 142.5) (end 119.44375 142.5) (width 0.2) (layer "F.Cu") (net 14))
 (via (at 119 142.5) (size 0.6) (drill 0.3) (layers "F.Cu" "B.Cu") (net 14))
 (via (at 80 140.5) (size 0.6) (drill 0.3) (layers "F.Cu" "B.Cu") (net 14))
 (segment (start 80 140.5) (end 117 140.5) (width 0.2) (layer "B.Cu") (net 14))
 (segment (start 117 140.5) (end 119 142.5) (width 0.2) (layer "B.Cu") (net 14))
 (segment (start 101.14375 128.35347) (end 86.24722 143.25) (width 0.2) (layer "F.Cu") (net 11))
 (segment (start 101.14375 124.2) (end 101.14375 128.35347) (width 0.2) (layer "F.Cu") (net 11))
 (segment (start 86.24722 143.25) (end 82.09375 143.25) (width 0.2) (layer "F.Cu") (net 11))
 (segment (start 97.64375 122.45) (end 97.64375 120.85625) (width 0.2) (layer "F.Cu") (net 3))
 (segment (start 142 123.5) (end 141.3 124.2) (width 0.2) (layer "F.Cu") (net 3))
 (segment (start 97.64375 120.85625) (end 98 120.5) (width 0.2) (layer "F.Cu") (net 3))
 (segment (start 141.3 124.2) (end 139.24375 124.2) (width 0.2) (layer "F.Cu") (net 3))
 (via (at 142 123.5) (size 0.6) (drill 0.3) (layers "F.Cu" "B.Cu") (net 3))
 (via (at 98 120.5) (size 0.6) (drill 0.3) (layers "F.Cu" "B.Cu") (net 3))
 (segment (start 98 120.5) (end 139 120.5) (width 0.2) (layer "B.Cu") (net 3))
 (segment (start 139 120.5) (end 142 123.5) (width 0.2) (layer "B.Cu") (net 3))
 (segment (start 123.316436 110.121) (end 124.717436 108.72) (width 0.2) (layer "F.Cu") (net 20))
 (segment (start 124.717436 108.72) (end 130.50875 108.72) (width 0.2) (layer "F.Cu") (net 20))
 (segment (start 110.05775 109.300314) (end 110.878436 110.121) (width 0.2) (layer "F.Cu") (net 20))
 (segment (start 110.878436 110.121) (end 123.316436 110.121) (width 0.2) (layer "F.Cu") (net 20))
 (segment (start 105.4675 90.5) (end 110.05775 95.09025) (width 0.2) (layer "F.Cu") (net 20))
 (segment (start 110.05775 95.09025) (end 110.05775 109.300314) (width 0.2) (layer "F.Cu") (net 20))
 (segment (start 105.4675 93.04) (end 109.65675 97.22925) (width 0.2) (layer "F.Cu") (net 6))
 (segment (start 109.65675 109.466414) (end 112.724228 112.533892) (width 0.2) (layer "F.Cu") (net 6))
 (segment (start 141 110.5) (end 142.78 108.72) (width 0.2) (layer "F.Cu") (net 6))
 (segment (start 142.78 108.72) (end 149.55875 108.72) (width 0.2) (layer "F.Cu") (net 6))
 (segment (start 123.578436 112.661) (end 124.739064 112.661) (width 0.2) (layer "F.Cu") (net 6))
 (segment (start 126.900064 110.5) (end 141 110.5) (width 0.2) (layer "F.Cu") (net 6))
 (segment (start 124.739064 112.661) (end 126.900064 110.5) (width 0.2) (layer "F.Cu") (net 6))
 (segment (start 112.724228 112.533892) (end 123.451328 112.533892) (width 0.2) (layer "F.Cu") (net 6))
 (segment (start 123.451328 112.533892) (end 123.578436 112.661) (width 0.2) (layer "F.Cu") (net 6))
 (segment (start 109.65675 97.22925) (end 109.65675 109.466414) (width 0.2) (layer "F.Cu") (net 6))
 (segment (start 126.27028 127.77) (end 130.50875 127.77) (width 0.2) (layer "F.Cu") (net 19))
 (segment (start 105.4675 95.58) (end 106.9845 97.097) (width 0.2) (layer "F.Cu") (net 19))
 (segment (start 106.9845 108.48422) (end 126.27028 127.77) (width 0.2) (layer "F.Cu") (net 19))
 (segment (start 106.9845 97.097) (end 106.9845 108.48422) (width 0.2) (layer "F.Cu") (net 19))
 (segment (start 105.4675 98.12) (end 106.56775 99.22025) (width 0.2) (layer "F.Cu") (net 18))
 (segment (start 106.56775 114.773816) (end 120.293934 128.5) (width 0.2) (layer "F.Cu") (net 18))
 (segment (start 106.56775 99.22025) (end 106.56775 114.773816) (width 0.2) (layer "F.Cu") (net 18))
 (segment (start 120.293934 128.5) (end 124 128.5) (width 0.2) (layer "F.Cu") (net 18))
 (via (at 124 128.5) (size 0.6) (drill 0.3) (layers "F.Cu" "B.Cu") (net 18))
 (segment (start 142.366436 129.171) (end 143.767436 127.77) (width 0.2) (layer "B.Cu") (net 18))
 (segment (start 143.767436 127.77) (end 149.55875 127.77) (width 0.2) (layer "B.Cu") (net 18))
 (segment (start 124 128.5) (end 125 128.5) (width 0.2) (layer "B.Cu") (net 18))
 (segment (start 125.671 129.171) (end 142.366436 129.171) (width 0.2) (layer "B.Cu") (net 18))
 (segment (start 125 128.5) (end 125.671 129.171) (width 0.2) (layer "B.Cu") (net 18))
 (segment (start 88.5575 82.88) (end 86.05875 85.37875) (width 0.2) (layer "F.Cu") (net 5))
 (segment (start 86.05875 85.37875) (end 86.05875 111.26) (width 0.2) (layer "F.Cu") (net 5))
 (segment (start 88.5575 85.42) (end 105.10875 101.97125) (width 0.2) (layer "F.Cu") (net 16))
 (segment (start 105.10875 101.97125) (end 105.10875 111.26) (width 0.2) (layer "F.Cu") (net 16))
 (segment (start 88.31487 87.96) (end 87 89.27487) (width 0.2) (layer "F.Cu") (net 13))
 (segment (start 87 110.219936) (end 87.45975 110.679686) (width 0.2) (layer "F.Cu") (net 13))
 (segment (start 87.45975 110.679686) (end 87.45975 128.909) (width 0.2) (layer "F.Cu") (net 13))
 (segment (start 87 89.27487) (end 87 110.219936) (width 0.2) (layer "F.Cu") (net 13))
 (segment (start 87.45975 128.909) (end 86.05875 130.31) (width 0.2) (layer "F.Cu") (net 13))
 (segment (start 89.3925 87.96) (end 88.31487 87.96) (width 0.2) (layer "F.Cu") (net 13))
 (segment (start 102.24475 103.35225) (end 102.24475 127.446) (width 0.2) (layer "F.Cu") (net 17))
 (segment (start 102.24475 127.446) (end 105.10875 130.31) (width 0.2) (layer "F.Cu") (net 17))
 (segment (start 89.3925 90.5) (end 102.24475 103.35225) (width 0.2) (layer "F.Cu") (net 17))
 (segment (start 118 95.4125) (end 118 102.099) (width 0.2) (layer "F.Cu") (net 4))
 (segment (start 116.69375 143.25) (end 115.96775 143.976) (width 0.2) (layer "F.Cu") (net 4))
 (segment (start 105.4675 82.88) (end 118 95.4125) (width 0.2) (layer "F.Cu") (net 4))
 (segment (start 79.31975 143.976) (end 78.59375 143.25) (width 0.2) (layer "F.Cu") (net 4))
 (segment (start 139.24375 122.45) (end 141.693566 122.45) (width 0.2) (layer "F.Cu") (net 4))
 (segment (start 141.693566 122.45) (end 151 113.143566) (width 0.2) (layer "F.Cu") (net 4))
 (segment (start 101.14375 122.45) (end 101.096875 122.403125) (width 0.2) (layer "F.Cu") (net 4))
 (segment (start 154.79375 143.25) (end 152.75 143.25) (width 0.2) (layer "F.Cu") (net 4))
 (segment (start 159 101.5) (end 158.29375 102.20625) (width 0.2) (layer "F.Cu") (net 4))
 (segment (start 118 102.099) (end 150 102.099) (width 0.2) (layer "F.Cu") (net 4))
 (segment (start 86.64275 135.201) (end 86.64275 132.751184) (width 0.2) (layer "F.Cu") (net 4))
 (segment (start 86.64275 132.751184) (end 88.894934 130.499) (width 0.2) (layer "F.Cu") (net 4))
 (segment (start 115.59275 104.126) (end 115.59275 102.674) (width 0.2) (layer "F.Cu") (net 4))
 (segment (start 150 102.099) (end 156.99275 102.099) (width 0.2) (layer "F.Cu") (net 4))
 (segment (start 116.16775 102.099) (end 118 102.099) (width 0.2) (layer "F.Cu") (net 4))
 (segment (start 158.29375 102.20625) (end 158.29375 103.4) (width 0.2) (layer "F.Cu") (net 4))
 (segment (start 119.46775 104.126) (end 115.59275 104.126) (width 0.2) (layer "F.Cu") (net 4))
 (segment (start 142.95 122.45) (end 143 122.5) (width 0.2) (layer "F.Cu") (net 4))
 (segment (start 115.96775 143.976) (end 79.31975 143.976) (width 0.2) (layer "F.Cu") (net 4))
 (segment (start 117.59522 143.25) (end 117.92261 143.57739) (width 0.2) (layer "F.Cu") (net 4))
 (segment (start 82.09375 103.4) (end 80 105.49375) (width 0.2) (layer "F.Cu") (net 4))
 (segment (start 150 90.8675) (end 150 102.099) (width 0.2) (layer "F.Cu") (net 4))
 (segment (start 115.59275 102.674) (end 116.16775 102.099) (width 0.2) (layer "F.Cu") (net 4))
 (segment (start 156.99275 102.099) (end 158.29375 103.4) (width 0.2) (layer "F.Cu") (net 4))
 (segment (start 80 105.49375) (end 80 107.5) (width 0.2) (layer "F.Cu") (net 4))
 (segment (start 88.894934 130.499) (end 93.09475 130.499) (width 0.2) (layer "F.Cu") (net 4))
 (segment (start 120.19375 103.4) (end 119.46775 104.126) (width 0.2) (layer "F.Cu") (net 4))
 (segment (start 93.09475 130.499) (end 101.14375 122.45) (width 0.2) (layer "F.Cu") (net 4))
 (segment (start 147.965 88.8325) (end 150 90.8675) (width 0.2) (layer "F.Cu") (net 4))
 (segment (start 78.59375 143.25) (end 86.64275 135.201) (width 0.2) (layer "F.Cu") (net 4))
 (segment (start 91 118.5) (end 97.19375 118.5) (width 0.2) (layer "F.Cu") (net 4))
 (segment (start 151 113.143566) (end 151 112.5) (width 0.2) (layer "F.Cu") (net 4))
 (segment (start 97.19375 118.5) (end 101.14375 122.45) (width 0.2) (layer "F.Cu") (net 4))
 (segment (start 116.69375 143.25) (end 117.59522 143.25) (width 0.2) (layer "F.Cu") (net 4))
 (segment (start 152.75 143.25) (end 152 142.5) (width 0.2) (layer "F.Cu") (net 4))
 (segment (start 139.24375 122.45) (end 142.95 122.45) (width 0.2) (layer "F.Cu") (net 4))
 (via (at 91 118.5) (size 0.6) (drill 0.3) (layers "F.Cu" "B.Cu") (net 4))
 (via (at 152 142.5) (size 0.6) (drill 0.3) (layers "F.Cu" "B.Cu") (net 4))
 (via (at 151 112.5) (size 0.6) (drill 0.3) (layers "F.Cu" "B.Cu") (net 4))
 (via (at 143 122.5) (size 0.6) (drill 0.3) (layers "F.Cu" "B.Cu") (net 4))
 (via (at 117.92261 143.57739) (size 0.6) (drill 0.3) (layers "F.Cu" "B.Cu") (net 4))
 (via (at 80 107.5) (size 0.6) (drill 0.3) (layers "F.Cu" "B.Cu") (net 4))
 (via (at 159 101.5) (size 0.6) (drill 0.3) (layers "F.Cu" "B.Cu") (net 4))
 (segment (start 117.92261 143.57739) (end 150.92261 143.57739) (width 0.2) (layer "B.Cu") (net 4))
 (segment (start 91 118.256066) (end 91 118.5) (width 0.2) (layer "B.Cu") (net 4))
 (segment (start 150.92261 143.57739) (end 152 142.5) (width 0.2) (layer "B.Cu") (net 4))
 (segment (start 159 104.5) (end 159 101.5) (width 0.2) (layer "B.Cu") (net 4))
 (segment (start 143 122.5) (end 157 122.5) (width 0.2) (layer "B.Cu") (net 4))
 (segment (start 80 107.5) (end 80.243934 107.5) (width 0.2) (layer "B.Cu") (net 4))
 (segment (start 157 137.5) (end 157 122.5) (width 0.2) (layer "B.Cu") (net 4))
 (segment (start 151 112.5) (end 159 104.5) (width 0.2) (layer "B.Cu") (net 4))
 (segment (start 152 142.5) (end 157 137.5) (width 0.2) (layer "B.Cu") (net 4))
 (segment (start 80.243934 107.5) (end 91 118.256066) (width 0.2) (layer "B.Cu") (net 4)))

